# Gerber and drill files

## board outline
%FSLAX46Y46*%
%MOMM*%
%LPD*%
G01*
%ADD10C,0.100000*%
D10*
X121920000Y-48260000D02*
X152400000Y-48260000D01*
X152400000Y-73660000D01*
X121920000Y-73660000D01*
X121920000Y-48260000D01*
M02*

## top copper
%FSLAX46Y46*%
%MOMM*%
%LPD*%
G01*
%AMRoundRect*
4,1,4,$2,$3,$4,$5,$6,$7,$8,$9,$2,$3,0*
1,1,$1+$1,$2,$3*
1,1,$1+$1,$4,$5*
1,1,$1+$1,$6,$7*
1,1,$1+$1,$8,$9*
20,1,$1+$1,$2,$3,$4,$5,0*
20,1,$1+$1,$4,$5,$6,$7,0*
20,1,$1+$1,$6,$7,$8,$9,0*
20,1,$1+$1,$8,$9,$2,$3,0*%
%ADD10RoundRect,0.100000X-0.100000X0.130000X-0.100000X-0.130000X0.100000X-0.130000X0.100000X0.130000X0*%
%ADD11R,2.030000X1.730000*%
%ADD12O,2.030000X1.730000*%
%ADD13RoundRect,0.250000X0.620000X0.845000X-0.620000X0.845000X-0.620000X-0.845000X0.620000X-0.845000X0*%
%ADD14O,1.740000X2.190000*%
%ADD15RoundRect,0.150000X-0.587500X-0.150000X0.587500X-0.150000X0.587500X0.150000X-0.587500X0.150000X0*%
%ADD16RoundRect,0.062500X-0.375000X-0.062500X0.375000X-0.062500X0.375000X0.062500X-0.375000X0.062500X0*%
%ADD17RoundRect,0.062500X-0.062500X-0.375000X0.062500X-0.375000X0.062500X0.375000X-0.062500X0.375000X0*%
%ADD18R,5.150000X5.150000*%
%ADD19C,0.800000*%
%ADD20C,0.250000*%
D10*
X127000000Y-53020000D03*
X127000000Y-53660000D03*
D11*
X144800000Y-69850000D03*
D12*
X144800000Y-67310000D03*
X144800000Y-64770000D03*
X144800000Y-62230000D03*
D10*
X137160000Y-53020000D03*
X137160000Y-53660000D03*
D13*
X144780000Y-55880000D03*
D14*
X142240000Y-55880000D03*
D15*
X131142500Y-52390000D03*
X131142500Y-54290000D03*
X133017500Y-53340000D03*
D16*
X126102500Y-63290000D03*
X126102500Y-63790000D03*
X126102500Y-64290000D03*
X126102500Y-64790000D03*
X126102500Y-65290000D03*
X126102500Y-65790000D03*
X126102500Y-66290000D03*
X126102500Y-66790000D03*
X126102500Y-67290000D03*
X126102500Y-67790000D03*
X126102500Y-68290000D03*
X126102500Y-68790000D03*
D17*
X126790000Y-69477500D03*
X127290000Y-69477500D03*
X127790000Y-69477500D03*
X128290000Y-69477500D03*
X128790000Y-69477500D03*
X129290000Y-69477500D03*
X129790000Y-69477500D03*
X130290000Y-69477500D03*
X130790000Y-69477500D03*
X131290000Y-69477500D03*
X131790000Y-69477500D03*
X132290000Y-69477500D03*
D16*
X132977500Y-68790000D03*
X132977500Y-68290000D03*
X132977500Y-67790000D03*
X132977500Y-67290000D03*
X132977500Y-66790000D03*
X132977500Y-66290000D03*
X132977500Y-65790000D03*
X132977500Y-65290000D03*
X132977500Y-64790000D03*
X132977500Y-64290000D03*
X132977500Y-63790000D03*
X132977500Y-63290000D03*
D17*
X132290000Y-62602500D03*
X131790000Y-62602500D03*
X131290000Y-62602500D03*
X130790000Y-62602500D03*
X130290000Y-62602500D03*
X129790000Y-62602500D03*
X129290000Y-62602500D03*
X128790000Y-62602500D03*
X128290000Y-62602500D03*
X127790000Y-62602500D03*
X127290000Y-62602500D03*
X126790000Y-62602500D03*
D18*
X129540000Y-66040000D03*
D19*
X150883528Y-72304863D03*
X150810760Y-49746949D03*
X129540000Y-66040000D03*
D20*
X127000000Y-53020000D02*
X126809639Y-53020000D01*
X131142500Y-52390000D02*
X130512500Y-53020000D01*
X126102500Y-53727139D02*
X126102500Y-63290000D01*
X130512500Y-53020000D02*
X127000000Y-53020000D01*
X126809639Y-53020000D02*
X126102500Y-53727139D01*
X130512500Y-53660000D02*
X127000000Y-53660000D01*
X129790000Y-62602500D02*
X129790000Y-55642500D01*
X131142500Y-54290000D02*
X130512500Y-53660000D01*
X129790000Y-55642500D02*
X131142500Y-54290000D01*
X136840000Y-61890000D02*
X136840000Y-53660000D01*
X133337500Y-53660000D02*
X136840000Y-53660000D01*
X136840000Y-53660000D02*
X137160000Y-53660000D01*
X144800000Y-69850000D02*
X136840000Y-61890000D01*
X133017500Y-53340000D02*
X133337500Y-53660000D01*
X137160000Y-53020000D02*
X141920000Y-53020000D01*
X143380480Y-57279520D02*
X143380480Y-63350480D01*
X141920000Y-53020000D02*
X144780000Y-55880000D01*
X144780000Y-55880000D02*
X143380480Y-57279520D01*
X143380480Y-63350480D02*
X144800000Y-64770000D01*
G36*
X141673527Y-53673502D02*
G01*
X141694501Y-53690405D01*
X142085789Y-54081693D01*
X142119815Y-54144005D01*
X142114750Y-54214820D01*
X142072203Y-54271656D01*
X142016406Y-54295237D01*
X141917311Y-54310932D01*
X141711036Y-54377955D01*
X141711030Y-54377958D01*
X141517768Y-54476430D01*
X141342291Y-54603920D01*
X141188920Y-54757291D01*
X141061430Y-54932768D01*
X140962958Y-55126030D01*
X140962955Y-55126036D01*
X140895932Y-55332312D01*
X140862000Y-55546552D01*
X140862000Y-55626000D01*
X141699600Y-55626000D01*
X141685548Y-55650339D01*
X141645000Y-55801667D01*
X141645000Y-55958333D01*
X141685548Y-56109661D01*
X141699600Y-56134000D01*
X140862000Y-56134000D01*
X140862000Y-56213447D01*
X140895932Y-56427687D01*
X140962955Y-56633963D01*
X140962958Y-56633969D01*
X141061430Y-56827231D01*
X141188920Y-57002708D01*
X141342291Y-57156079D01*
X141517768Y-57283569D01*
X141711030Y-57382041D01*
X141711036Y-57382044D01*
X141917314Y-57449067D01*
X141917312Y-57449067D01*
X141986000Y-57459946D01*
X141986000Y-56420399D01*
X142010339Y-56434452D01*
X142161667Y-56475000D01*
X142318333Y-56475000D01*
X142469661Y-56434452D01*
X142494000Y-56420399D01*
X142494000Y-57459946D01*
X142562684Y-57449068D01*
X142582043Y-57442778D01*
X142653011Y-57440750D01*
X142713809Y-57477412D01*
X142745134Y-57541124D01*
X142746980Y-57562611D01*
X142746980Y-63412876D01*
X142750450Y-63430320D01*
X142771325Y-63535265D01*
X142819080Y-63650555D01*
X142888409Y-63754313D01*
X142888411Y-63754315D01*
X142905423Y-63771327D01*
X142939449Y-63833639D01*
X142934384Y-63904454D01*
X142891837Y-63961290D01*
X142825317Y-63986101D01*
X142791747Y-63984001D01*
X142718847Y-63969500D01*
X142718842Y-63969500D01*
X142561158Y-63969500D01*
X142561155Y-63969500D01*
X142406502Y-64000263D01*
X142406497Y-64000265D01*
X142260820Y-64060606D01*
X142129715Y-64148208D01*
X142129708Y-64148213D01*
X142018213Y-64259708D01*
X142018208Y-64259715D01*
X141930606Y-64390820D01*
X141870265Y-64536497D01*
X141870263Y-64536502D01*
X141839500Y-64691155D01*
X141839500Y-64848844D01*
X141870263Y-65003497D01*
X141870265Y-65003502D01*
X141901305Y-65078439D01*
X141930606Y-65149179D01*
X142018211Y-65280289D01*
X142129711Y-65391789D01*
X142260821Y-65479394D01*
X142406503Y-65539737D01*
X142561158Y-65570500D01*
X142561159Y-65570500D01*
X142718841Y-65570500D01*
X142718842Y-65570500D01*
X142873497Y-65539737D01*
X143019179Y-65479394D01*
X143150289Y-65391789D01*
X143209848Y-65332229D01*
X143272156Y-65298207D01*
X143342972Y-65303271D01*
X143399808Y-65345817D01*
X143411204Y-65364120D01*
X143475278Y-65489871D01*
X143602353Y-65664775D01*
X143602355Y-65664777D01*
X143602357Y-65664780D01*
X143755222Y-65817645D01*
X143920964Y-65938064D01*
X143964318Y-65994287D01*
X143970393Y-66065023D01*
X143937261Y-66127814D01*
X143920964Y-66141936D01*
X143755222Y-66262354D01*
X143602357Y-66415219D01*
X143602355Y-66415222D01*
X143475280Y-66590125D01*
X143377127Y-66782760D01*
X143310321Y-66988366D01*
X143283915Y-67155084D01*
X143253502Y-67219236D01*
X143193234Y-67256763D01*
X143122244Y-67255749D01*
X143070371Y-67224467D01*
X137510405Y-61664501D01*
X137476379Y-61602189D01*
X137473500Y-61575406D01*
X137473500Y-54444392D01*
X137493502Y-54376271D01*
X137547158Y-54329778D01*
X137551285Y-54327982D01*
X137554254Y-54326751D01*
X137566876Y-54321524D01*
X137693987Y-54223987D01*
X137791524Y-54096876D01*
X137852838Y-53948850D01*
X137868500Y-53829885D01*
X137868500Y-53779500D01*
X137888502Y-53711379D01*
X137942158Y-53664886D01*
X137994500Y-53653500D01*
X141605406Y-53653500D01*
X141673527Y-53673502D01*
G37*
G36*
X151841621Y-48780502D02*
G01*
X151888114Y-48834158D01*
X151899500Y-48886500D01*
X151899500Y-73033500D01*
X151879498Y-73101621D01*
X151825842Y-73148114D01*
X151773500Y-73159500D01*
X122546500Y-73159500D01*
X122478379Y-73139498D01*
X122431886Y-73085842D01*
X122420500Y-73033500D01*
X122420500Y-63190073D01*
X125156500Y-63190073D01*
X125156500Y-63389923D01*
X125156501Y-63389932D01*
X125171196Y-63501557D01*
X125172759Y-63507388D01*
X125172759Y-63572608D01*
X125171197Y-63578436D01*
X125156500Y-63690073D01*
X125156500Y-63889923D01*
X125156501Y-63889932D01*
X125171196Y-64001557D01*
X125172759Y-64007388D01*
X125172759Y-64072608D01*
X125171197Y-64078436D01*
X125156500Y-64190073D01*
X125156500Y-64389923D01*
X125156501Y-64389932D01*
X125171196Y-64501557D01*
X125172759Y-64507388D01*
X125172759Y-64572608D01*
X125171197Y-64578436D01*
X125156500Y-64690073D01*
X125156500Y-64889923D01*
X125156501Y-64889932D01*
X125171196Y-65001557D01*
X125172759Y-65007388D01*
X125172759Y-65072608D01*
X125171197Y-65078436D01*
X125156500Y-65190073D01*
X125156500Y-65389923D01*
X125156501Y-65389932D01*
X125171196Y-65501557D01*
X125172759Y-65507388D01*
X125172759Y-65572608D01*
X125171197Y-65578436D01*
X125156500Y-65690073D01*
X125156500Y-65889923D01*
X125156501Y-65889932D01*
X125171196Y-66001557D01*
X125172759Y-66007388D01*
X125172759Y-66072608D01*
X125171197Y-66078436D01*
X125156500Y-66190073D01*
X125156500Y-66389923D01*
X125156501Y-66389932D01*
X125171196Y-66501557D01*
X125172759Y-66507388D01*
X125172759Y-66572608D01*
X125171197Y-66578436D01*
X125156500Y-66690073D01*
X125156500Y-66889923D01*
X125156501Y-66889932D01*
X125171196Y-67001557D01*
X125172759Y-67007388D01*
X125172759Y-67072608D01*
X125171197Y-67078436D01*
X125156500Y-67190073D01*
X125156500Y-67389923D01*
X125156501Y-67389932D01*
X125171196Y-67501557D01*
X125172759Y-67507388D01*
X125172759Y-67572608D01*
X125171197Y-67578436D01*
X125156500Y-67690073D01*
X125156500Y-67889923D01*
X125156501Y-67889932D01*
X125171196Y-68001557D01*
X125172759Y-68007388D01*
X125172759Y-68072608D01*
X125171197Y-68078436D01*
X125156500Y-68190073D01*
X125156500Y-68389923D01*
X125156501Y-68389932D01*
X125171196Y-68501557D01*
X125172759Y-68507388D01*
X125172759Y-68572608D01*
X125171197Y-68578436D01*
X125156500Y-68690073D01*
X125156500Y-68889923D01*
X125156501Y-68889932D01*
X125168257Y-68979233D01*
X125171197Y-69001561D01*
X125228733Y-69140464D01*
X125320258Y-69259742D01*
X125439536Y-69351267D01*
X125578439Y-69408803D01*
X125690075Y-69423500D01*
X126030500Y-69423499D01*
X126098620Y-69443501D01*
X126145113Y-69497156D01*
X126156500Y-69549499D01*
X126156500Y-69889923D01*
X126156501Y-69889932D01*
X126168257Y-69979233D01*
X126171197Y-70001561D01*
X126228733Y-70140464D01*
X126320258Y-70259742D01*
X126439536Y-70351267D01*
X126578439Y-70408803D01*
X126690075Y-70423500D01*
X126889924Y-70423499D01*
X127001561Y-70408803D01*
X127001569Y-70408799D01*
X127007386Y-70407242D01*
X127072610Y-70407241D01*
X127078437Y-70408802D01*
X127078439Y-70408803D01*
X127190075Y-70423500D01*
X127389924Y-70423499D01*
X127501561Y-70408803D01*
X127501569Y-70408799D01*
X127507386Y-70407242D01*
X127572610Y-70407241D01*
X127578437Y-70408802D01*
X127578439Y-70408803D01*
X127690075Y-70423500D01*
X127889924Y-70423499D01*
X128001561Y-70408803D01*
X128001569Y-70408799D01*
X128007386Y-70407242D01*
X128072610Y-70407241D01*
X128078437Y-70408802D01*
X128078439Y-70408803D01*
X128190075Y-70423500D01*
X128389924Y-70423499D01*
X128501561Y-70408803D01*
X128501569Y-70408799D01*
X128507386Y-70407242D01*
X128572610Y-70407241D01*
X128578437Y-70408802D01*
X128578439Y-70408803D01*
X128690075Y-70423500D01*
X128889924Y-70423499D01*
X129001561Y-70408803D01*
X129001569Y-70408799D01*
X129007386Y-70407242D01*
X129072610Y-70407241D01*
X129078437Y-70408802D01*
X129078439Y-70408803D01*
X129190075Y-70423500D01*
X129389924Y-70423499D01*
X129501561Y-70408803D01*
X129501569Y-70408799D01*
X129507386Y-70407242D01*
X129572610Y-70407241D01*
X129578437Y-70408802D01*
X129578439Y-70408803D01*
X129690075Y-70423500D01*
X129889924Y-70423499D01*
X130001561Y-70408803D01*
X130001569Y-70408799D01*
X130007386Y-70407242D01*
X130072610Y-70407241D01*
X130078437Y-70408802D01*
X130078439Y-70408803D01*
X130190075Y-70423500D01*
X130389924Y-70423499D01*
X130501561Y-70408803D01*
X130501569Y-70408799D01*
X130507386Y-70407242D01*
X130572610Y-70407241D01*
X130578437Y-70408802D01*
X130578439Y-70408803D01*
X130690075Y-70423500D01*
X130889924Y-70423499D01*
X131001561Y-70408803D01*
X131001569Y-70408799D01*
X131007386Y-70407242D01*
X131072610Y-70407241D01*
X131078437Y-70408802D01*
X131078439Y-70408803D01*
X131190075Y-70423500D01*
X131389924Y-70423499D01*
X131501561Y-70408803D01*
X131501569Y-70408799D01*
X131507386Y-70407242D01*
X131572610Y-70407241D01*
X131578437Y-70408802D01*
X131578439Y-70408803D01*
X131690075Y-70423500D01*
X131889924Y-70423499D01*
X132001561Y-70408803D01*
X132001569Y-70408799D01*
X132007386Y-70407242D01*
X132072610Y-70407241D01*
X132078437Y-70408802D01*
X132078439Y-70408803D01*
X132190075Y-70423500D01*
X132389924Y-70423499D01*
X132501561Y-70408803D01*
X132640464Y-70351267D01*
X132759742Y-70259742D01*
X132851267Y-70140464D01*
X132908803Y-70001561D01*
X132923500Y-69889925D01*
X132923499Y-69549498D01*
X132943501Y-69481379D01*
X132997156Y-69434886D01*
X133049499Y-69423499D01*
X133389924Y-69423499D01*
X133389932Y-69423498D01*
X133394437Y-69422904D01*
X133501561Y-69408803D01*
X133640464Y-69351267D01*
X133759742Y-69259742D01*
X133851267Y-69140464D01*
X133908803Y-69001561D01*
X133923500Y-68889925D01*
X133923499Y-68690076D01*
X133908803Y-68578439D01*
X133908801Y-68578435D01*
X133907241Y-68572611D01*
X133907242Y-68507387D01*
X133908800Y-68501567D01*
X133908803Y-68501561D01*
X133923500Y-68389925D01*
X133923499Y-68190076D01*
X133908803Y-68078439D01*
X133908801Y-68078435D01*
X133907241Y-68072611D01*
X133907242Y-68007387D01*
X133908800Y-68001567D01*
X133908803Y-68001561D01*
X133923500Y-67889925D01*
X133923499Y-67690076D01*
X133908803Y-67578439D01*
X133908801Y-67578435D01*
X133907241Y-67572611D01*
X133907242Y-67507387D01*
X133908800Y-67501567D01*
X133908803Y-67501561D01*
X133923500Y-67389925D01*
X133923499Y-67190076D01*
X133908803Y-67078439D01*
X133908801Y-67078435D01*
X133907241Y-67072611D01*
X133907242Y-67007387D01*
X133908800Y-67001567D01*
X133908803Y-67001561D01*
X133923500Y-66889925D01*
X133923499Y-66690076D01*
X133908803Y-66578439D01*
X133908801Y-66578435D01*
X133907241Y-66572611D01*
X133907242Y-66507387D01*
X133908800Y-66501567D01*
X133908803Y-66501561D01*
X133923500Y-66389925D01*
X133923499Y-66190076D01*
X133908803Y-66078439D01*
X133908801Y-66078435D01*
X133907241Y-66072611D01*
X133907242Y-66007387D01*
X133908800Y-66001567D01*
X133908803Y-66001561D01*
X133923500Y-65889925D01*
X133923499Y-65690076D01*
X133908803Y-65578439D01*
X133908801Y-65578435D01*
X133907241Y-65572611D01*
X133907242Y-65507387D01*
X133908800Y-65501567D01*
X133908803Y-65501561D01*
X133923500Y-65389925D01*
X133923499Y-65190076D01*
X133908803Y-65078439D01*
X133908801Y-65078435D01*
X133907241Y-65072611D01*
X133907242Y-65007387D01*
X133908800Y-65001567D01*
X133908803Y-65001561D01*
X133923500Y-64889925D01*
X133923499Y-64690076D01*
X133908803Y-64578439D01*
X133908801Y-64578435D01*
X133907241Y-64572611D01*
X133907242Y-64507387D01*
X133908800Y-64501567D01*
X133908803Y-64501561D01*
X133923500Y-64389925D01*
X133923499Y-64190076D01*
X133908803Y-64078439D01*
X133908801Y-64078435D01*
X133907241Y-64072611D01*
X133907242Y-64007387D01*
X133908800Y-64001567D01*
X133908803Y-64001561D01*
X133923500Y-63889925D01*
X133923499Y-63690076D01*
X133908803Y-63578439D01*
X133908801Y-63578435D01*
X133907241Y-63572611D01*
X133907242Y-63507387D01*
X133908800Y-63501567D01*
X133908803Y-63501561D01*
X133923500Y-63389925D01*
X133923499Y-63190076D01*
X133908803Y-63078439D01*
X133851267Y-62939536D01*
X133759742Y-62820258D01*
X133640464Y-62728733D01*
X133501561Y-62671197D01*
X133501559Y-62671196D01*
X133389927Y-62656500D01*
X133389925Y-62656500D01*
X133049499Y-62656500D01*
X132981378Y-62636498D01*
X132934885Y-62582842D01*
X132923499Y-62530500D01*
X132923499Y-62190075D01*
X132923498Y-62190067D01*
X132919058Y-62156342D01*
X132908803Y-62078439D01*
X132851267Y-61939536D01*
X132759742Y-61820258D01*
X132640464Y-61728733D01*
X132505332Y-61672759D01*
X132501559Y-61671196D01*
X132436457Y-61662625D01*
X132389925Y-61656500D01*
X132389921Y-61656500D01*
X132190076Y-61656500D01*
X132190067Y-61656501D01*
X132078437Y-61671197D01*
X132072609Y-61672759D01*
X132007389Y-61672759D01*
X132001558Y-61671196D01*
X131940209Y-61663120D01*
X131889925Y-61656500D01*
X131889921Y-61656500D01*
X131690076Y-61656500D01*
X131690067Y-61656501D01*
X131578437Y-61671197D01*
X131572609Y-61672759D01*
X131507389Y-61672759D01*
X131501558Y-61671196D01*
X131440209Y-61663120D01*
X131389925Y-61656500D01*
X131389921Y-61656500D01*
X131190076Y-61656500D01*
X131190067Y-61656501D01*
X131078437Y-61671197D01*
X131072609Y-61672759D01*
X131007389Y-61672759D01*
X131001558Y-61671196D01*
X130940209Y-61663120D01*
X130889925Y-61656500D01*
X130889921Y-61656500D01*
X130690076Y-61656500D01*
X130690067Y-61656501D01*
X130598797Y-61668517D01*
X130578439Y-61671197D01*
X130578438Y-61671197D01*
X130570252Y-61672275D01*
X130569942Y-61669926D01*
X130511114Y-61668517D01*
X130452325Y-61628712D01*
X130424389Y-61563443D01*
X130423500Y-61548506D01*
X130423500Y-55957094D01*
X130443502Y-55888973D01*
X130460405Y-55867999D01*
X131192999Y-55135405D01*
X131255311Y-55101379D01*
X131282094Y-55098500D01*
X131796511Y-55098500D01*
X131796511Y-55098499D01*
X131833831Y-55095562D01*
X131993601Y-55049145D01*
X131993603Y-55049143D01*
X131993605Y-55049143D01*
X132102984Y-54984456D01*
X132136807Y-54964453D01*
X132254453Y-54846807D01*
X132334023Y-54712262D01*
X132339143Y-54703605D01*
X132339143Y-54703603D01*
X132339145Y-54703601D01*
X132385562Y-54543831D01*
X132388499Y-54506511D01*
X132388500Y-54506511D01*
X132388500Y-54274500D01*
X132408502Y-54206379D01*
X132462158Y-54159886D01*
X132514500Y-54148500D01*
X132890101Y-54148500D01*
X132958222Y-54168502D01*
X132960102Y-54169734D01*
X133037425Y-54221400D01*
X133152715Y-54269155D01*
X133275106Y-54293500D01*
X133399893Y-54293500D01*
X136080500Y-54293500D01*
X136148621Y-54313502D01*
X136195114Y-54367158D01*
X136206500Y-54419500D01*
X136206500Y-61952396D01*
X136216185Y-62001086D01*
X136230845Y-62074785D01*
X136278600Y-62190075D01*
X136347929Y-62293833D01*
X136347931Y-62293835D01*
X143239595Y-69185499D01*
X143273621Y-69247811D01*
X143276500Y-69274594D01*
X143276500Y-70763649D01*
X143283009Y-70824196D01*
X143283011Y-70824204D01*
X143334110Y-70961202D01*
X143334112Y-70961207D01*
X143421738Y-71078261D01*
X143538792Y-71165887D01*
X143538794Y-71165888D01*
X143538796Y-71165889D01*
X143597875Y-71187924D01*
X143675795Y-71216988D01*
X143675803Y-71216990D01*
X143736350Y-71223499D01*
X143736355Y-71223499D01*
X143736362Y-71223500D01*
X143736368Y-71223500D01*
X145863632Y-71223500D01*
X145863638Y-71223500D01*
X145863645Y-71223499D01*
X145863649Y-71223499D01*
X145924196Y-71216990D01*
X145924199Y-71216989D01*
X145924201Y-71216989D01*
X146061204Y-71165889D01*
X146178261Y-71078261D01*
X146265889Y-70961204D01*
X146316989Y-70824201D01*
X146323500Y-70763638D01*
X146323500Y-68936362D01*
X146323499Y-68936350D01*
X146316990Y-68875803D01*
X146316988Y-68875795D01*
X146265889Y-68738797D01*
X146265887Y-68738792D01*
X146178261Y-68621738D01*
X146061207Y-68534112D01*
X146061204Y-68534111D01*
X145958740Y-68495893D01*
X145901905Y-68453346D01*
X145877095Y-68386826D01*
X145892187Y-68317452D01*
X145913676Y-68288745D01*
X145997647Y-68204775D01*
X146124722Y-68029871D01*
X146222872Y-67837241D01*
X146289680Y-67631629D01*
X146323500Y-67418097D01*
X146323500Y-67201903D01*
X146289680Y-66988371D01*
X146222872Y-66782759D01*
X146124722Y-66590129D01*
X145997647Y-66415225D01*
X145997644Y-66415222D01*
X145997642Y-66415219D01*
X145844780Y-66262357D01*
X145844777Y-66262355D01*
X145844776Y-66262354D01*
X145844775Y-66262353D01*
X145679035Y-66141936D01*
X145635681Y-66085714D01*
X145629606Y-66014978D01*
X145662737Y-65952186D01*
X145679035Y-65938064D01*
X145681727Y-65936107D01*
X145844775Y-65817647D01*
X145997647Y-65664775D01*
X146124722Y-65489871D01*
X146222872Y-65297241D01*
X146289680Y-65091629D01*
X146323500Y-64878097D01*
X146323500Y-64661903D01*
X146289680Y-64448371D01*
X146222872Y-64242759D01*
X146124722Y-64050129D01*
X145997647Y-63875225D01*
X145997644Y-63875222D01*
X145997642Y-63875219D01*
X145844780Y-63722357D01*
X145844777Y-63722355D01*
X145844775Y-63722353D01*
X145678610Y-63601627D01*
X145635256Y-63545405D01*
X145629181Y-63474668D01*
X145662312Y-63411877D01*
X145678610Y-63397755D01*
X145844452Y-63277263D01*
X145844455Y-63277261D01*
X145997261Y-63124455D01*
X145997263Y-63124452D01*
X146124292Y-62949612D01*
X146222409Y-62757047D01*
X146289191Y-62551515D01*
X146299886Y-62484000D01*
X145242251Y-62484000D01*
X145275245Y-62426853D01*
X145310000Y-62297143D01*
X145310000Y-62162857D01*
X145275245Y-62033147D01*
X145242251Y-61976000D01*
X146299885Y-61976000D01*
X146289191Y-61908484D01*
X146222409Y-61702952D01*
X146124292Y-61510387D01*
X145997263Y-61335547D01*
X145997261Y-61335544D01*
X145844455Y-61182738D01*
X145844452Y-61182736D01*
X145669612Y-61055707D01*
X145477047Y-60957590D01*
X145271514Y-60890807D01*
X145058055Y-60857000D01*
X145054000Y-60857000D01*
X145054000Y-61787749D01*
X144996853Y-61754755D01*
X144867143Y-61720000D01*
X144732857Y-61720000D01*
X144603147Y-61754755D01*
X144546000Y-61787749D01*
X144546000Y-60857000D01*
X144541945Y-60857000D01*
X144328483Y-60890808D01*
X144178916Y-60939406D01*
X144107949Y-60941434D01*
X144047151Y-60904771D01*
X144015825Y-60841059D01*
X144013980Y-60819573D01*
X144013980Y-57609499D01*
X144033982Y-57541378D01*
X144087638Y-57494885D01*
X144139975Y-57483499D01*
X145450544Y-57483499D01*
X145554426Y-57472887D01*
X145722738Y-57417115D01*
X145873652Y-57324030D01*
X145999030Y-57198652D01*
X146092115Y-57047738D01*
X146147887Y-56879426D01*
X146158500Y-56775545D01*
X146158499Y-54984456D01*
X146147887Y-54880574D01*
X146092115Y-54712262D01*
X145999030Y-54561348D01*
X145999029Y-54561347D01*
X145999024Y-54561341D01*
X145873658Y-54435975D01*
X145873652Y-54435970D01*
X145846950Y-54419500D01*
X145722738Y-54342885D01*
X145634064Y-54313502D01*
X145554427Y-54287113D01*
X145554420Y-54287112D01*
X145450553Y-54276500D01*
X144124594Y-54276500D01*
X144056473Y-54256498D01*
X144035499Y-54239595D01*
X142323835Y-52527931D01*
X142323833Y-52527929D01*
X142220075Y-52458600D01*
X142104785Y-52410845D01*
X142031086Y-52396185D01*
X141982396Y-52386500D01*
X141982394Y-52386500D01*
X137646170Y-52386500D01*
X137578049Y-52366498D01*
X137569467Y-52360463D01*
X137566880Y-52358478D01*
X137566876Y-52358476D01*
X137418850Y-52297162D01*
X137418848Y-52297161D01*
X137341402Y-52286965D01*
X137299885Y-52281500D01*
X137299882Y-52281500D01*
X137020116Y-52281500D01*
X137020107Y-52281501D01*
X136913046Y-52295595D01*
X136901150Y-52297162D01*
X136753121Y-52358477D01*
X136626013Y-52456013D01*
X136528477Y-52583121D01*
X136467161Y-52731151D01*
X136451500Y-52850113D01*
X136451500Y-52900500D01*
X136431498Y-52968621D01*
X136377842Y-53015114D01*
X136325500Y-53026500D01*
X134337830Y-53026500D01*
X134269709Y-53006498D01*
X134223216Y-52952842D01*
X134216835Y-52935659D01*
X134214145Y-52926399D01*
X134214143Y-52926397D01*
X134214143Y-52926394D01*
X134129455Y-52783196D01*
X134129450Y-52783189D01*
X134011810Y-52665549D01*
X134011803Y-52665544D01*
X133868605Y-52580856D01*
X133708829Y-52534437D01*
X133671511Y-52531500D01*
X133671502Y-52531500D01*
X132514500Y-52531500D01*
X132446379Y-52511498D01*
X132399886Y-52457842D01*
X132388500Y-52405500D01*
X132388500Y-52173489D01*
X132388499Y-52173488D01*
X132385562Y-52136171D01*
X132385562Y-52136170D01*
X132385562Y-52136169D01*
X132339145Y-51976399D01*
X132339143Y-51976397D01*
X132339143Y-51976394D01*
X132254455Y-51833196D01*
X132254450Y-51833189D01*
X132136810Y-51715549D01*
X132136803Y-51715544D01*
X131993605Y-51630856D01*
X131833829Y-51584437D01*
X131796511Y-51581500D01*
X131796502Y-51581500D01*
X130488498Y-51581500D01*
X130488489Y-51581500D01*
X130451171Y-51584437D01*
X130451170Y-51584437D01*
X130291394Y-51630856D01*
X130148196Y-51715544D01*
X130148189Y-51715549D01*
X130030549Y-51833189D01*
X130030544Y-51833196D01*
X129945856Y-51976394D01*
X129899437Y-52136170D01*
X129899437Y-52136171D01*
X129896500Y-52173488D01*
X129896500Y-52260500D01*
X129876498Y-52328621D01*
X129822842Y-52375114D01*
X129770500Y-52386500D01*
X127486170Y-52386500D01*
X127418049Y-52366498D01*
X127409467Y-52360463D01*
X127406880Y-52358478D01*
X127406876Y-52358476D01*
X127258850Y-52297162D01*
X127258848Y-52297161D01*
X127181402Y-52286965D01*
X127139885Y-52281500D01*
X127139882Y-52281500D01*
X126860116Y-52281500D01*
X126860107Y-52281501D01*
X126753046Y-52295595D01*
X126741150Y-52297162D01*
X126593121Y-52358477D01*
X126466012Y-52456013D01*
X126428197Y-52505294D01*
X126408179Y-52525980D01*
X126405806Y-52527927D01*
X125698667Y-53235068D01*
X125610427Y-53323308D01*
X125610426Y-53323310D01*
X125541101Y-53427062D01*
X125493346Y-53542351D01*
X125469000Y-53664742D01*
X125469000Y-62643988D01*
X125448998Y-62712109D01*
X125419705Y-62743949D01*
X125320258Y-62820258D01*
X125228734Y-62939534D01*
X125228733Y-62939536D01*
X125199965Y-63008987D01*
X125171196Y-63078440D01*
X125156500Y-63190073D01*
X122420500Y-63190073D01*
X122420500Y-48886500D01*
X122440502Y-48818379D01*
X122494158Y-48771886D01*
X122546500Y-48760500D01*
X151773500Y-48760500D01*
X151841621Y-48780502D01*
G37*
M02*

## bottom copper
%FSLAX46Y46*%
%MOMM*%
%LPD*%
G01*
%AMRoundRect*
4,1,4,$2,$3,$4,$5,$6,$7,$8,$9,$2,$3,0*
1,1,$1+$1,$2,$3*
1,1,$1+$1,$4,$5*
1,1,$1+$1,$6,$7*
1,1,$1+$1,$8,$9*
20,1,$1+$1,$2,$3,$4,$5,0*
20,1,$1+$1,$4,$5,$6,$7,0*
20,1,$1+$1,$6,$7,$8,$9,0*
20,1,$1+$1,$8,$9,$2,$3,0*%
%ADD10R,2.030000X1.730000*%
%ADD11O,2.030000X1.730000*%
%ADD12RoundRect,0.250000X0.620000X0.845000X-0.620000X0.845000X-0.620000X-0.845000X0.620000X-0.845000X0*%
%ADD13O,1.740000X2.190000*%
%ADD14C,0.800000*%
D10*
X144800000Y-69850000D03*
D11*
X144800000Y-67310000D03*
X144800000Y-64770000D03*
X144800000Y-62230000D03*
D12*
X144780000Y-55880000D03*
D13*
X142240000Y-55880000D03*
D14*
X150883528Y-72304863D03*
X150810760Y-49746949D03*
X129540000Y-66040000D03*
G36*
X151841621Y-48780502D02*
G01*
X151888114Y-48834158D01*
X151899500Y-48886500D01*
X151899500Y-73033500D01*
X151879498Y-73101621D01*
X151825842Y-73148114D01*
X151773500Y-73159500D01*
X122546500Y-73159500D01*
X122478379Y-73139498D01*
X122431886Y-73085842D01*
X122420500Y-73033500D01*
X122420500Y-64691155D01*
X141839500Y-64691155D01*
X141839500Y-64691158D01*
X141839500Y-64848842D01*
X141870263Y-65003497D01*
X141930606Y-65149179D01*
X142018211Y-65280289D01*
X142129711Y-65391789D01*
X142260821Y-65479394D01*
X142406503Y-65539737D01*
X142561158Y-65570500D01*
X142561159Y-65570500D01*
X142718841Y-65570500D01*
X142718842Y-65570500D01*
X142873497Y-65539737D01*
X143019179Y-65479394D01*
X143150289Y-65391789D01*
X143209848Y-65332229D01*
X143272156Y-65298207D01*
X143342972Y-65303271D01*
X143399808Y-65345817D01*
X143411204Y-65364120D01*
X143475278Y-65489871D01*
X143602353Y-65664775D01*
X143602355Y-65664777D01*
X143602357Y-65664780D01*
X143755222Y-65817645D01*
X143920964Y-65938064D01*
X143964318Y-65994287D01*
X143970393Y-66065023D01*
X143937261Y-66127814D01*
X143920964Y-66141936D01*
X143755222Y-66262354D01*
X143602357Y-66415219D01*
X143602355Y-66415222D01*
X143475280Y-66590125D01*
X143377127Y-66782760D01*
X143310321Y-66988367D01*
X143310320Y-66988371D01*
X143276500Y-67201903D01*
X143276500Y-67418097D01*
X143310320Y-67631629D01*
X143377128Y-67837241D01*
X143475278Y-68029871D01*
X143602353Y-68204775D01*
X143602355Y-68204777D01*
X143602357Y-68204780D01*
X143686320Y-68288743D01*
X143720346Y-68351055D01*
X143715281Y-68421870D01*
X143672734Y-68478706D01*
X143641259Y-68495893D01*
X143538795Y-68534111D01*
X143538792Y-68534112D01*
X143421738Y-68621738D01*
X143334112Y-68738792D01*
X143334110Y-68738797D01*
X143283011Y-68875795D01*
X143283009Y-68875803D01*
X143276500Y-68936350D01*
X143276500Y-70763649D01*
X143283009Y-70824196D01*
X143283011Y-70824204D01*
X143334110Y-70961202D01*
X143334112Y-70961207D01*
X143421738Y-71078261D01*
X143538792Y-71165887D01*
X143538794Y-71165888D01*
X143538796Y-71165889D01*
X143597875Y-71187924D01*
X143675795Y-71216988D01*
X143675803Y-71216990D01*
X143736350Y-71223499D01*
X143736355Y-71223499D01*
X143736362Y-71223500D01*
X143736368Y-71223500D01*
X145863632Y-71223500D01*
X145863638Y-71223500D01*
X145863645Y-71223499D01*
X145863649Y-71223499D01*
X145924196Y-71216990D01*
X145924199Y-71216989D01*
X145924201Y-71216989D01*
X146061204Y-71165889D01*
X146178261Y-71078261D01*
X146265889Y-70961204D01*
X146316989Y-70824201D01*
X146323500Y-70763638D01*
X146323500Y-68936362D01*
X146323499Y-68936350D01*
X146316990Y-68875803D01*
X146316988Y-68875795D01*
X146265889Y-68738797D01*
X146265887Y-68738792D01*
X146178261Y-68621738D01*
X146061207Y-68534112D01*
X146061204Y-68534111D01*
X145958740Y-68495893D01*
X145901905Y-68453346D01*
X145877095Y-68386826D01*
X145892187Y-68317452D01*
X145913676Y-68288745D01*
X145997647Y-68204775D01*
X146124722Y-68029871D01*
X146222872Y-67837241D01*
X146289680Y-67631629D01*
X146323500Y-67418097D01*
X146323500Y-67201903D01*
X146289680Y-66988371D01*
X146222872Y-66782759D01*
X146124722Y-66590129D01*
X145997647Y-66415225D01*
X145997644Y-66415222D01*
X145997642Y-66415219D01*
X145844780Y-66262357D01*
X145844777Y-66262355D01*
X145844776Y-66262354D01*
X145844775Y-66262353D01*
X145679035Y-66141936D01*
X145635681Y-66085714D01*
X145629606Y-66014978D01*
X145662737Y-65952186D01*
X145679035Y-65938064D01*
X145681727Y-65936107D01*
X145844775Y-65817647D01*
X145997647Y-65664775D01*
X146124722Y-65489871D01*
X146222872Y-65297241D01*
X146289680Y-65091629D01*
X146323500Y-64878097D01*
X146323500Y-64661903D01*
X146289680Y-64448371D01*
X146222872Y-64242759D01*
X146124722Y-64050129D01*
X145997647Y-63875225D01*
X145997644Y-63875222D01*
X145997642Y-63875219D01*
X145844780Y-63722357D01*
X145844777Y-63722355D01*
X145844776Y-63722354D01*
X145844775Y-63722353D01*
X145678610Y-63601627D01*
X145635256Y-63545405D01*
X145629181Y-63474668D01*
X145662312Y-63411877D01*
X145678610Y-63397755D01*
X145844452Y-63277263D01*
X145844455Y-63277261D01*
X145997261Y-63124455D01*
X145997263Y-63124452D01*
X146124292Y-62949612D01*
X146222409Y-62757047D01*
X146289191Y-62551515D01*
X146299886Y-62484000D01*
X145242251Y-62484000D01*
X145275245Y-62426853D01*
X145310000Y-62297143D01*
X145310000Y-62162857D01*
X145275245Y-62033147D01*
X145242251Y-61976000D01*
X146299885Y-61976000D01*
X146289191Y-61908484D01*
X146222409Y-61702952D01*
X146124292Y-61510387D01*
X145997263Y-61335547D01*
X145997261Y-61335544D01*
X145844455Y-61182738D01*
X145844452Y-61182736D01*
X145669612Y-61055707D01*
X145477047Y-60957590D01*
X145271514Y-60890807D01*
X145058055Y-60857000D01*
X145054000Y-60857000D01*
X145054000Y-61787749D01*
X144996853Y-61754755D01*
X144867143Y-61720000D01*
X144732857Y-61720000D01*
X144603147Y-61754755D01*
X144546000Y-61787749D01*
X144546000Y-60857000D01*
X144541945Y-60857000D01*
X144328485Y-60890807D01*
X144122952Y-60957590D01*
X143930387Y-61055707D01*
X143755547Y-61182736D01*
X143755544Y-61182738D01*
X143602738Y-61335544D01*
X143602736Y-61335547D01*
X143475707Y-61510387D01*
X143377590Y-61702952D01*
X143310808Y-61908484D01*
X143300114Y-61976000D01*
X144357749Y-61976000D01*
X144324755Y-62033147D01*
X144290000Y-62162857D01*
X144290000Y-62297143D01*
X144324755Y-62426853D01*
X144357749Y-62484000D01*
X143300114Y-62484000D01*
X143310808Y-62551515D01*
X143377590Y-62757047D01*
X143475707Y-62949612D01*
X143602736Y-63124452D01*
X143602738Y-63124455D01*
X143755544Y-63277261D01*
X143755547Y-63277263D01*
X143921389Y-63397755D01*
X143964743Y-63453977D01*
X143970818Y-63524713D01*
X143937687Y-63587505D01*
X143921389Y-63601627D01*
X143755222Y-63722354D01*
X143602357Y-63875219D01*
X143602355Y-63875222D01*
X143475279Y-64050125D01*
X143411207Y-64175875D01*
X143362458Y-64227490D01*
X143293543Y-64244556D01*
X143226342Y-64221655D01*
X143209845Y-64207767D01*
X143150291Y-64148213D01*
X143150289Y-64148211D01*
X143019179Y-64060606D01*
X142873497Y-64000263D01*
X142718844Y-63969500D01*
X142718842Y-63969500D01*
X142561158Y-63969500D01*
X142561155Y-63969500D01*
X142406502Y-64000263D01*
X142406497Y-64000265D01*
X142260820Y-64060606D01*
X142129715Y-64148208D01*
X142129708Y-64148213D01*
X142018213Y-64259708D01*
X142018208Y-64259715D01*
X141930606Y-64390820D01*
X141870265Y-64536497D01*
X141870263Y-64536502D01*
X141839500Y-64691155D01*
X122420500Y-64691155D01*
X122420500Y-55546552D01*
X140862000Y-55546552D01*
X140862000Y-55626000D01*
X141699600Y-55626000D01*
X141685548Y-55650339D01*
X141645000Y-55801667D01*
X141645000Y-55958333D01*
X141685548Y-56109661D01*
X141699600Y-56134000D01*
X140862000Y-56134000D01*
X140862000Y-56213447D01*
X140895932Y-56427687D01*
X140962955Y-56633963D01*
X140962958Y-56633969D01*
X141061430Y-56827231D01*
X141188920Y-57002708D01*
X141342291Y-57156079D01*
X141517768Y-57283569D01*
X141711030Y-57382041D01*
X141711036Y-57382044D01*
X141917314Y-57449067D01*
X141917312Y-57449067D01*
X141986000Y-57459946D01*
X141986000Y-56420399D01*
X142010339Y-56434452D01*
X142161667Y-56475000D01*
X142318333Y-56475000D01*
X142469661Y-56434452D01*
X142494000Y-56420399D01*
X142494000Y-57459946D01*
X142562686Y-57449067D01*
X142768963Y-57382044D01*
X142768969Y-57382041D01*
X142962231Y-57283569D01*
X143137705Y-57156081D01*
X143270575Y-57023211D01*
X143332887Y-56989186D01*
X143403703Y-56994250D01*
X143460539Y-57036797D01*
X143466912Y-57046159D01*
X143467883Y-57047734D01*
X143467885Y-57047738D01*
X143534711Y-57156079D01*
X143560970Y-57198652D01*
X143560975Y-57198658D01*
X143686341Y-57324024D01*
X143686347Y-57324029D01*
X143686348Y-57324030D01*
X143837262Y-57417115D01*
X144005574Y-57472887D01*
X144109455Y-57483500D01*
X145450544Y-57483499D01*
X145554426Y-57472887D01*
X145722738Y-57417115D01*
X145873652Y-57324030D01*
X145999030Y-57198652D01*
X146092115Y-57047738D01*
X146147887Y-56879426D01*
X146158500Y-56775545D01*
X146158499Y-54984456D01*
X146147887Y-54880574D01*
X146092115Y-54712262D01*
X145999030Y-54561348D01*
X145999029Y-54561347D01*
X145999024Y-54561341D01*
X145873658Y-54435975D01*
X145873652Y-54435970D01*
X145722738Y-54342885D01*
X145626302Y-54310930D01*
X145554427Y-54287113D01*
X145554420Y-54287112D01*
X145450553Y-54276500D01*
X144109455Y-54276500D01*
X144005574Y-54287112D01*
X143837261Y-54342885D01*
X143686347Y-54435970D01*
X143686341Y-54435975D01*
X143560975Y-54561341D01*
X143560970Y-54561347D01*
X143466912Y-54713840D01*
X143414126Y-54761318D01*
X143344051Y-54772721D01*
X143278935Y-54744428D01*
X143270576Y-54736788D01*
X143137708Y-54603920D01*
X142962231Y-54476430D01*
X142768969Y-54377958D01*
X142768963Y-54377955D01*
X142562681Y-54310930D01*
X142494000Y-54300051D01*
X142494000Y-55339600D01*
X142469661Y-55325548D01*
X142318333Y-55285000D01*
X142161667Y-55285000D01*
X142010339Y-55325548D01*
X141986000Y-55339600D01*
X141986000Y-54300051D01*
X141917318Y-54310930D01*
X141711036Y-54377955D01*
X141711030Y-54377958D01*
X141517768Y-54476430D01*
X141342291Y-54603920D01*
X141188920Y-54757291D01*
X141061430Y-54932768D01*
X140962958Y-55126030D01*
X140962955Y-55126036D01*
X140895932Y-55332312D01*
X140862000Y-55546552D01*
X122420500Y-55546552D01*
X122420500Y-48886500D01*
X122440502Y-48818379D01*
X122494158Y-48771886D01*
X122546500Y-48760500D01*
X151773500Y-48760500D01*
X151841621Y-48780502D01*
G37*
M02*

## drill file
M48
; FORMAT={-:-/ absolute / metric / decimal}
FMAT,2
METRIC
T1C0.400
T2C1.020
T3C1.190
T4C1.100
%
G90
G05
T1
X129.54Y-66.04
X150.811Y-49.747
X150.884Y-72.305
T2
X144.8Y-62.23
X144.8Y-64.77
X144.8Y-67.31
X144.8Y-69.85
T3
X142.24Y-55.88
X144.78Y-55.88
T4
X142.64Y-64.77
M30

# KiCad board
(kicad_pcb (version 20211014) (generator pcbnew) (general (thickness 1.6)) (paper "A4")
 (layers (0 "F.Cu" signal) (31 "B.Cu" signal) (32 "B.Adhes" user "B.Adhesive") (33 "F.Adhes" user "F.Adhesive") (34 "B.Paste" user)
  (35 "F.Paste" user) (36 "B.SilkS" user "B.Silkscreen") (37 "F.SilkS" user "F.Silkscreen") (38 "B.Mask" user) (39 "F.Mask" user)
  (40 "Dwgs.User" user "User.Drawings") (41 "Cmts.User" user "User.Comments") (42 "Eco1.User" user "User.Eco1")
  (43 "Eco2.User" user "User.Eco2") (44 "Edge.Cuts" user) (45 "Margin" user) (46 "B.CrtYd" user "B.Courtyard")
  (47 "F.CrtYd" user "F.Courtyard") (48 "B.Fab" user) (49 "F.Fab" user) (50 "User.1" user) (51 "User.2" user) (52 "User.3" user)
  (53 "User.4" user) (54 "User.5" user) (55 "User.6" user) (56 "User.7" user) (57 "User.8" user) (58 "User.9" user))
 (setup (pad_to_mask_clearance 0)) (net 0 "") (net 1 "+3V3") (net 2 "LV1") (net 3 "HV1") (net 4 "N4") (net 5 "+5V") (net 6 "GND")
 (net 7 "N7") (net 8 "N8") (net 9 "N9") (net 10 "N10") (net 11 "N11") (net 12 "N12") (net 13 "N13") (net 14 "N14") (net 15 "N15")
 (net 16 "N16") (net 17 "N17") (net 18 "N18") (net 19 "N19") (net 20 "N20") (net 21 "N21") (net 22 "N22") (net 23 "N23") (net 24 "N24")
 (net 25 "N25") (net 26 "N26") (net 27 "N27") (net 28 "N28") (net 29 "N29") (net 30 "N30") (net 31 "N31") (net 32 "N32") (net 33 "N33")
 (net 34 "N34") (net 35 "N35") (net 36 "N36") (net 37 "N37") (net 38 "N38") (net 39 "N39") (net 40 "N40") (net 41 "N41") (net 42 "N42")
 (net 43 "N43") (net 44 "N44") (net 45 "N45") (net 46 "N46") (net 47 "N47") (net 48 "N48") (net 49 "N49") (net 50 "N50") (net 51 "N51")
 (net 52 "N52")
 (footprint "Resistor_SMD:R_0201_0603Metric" (layer "F.Cu") (at 127 53.34 -90)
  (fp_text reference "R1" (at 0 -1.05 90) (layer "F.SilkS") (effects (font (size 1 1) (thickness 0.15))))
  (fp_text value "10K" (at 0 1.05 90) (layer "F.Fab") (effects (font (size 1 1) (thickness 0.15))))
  (pad "" smd roundrect locked (at 0.345 0 270) (size 0.318 0.36) (layers "F.Paste") (roundrect_rratio 0.25))
  (pad "" smd roundrect locked (at -0.345 0 270) (size 0.318 0.36) (layers "F.Paste") (roundrect_rratio 0.25))
  (pad "1" smd roundrect locked (at -0.32 0 270) (size 0.46 0.4) (layers "F.Cu" "F.Mask") (roundrect_rratio 0.25) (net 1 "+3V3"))
  (pad "2" smd roundrect locked (at 0.32 0 270) (size 0.46 0.4) (layers "F.Cu" "F.Mask") (roundrect_rratio 0.25) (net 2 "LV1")))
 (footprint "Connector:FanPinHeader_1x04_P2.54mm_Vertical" (layer "F.Cu") (at 144.8 69.85 90)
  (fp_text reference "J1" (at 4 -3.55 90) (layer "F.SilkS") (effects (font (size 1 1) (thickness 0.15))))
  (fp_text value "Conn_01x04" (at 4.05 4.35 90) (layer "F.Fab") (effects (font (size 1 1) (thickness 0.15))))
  (pad "" np_thru_hole circle locked (at 5.08 -2.16 180) (size 1.1 1.1) (drill 1.1) (layers *.Cu *.Mask))
  (pad "1" thru_hole rect locked (at 0 0 180) (size 2.03 1.73) (drill 1.02) (layers *.Cu *.Mask) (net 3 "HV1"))
  (pad "2" thru_hole oval locked (at 2.54 0 180) (size 2.03 1.73) (drill 1.02) (layers *.Cu *.Mask) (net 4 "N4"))
  (pad "3" thru_hole oval locked (at 5.08 0 180) (size 2.03 1.73) (drill 1.02) (layers *.Cu *.Mask) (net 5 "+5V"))
  (pad "4" thru_hole oval locked (at 7.62 0 180) (size 2.03 1.73) (drill 1.02) (layers *.Cu *.Mask) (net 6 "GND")))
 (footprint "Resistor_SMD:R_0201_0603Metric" (layer "F.Cu") (at 137.16 53.34 -90)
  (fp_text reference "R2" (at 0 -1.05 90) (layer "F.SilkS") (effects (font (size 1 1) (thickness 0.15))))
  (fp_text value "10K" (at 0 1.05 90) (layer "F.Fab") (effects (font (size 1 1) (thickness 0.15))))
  (pad "" smd roundrect locked (at 0.345 0 270) (size 0.318 0.36) (layers "F.Paste") (roundrect_rratio 0.25))
  (pad "" smd roundrect locked (at -0.345 0 270) (size 0.318 0.36) (layers "F.Paste") (roundrect_rratio 0.25))
  (pad "1" smd roundrect locked (at -0.32 0 270) (size 0.46 0.4) (layers "F.Cu" "F.Mask") (roundrect_rratio 0.25) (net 5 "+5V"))
  (pad "2" smd roundrect locked (at 0.32 0 270) (size 0.46 0.4) (layers "F.Cu" "F.Mask") (roundrect_rratio 0.25) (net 3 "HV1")))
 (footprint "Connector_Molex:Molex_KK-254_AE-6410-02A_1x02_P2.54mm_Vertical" (layer "F.Cu") (at 144.78 55.88 180)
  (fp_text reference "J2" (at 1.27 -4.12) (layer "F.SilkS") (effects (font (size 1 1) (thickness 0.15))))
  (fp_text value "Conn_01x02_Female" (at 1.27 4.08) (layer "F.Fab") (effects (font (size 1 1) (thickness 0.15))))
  (pad "1" thru_hole roundrect locked (at 0 0 180) (size 1.74 2.19) (drill 1.19) (layers *.Cu *.Mask) (roundrect_rratio 0.143678)
   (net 5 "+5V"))
  (pad "2" thru_hole oval locked (at 2.54 0 180) (size 1.74 2.19) (drill 1.19) (layers *.Cu *.Mask) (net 6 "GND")))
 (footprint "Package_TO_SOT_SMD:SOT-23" (layer "F.Cu") (at 132.08 53.34)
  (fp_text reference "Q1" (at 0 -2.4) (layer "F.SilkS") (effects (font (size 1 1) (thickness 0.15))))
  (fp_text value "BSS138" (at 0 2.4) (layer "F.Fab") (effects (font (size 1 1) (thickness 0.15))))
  (pad "1" smd roundrect locked (at -0.9375 -0.95) (size 1.475 0.6) (layers "F.Cu" "F.Paste" "F.Mask") (roundrect_rratio 0.25)
   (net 1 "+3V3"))
  (pad "2" smd roundrect locked (at -0.9375 0.95) (size 1.475 0.6) (layers "F.Cu" "F.Paste" "F.Mask") (roundrect_rratio 0.25) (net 2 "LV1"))
  (pad "3" smd roundrect locked (at 0.9375 0) (size 1.475 0.6) (layers "F.Cu" "F.Paste" "F.Mask") (roundrect_rratio 0.25) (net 3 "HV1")))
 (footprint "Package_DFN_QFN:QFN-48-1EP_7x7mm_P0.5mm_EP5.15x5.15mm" (layer "F.Cu") (at 129.54 66.04)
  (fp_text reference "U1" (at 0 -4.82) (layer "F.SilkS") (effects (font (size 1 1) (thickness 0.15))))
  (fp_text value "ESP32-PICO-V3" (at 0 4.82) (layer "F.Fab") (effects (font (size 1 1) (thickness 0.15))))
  (pad "" smd roundrect locked (at -1.935 -0.645) (size 1.04 1.04) (layers "F.Paste") (roundrect_rratio 0.240385))
  (pad "" smd roundrect locked (at 1.935 1.935) (size 1.04 1.04) (layers "F.Paste") (roundrect_rratio 0.240385))
  (pad "" smd roundrect locked (at 0.645 0.645) (size 1.04 1.04) (layers "F.Paste") (roundrect_rratio 0.240385))
  (pad "" smd roundrect locked (at -1.935 1.935) (size 1.04 1.04) (layers "F.Paste") (roundrect_rratio 0.240385))
  (pad "" smd roundrect locked (at 1.935 -0.645) (size 1.04 1.04) (layers "F.Paste") (roundrect_rratio 0.240385))
  (pad "" smd roundrect locked (at -0.645 -1.935) (size 1.04 1.04) (layers "F.Paste") (roundrect_rratio 0.240385))
  (pad "" smd roundrect locked (at -0.645 -0.645) (size 1.04 1.04) (layers "F.Paste") (roundrect_rratio 0.240385))
  (pad "" smd roundrect locked (at 1.935 0.645) (size 1.04 1.04) (layers "F.Paste") (roundrect_rratio 0.240385))
  (pad "" smd roundrect locked (at -1.935 0.645) (size 1.04 1.04) (layers "F.Paste") (roundrect_rratio 0.240385))
  (pad "" smd roundrect locked (at 0.645 1.935) (size 1.04 1.04) (layers "F.Paste") (roundrect_rratio 0.240385))
  (pad "" smd roundrect locked (at -0.645 0.645) (size 1.04 1.04) (layers "F.Paste") (roundrect_rratio 0.240385))
  (pad "" smd roundrect locked (at 0.645 -0.645) (size 1.04 1.04) (layers "F.Paste") (roundrect_rratio 0.240385))
  (pad "" smd roundrect locked (at 0.645 -1.935) (size 1.04 1.04) (layers "F.Paste") (roundrect_rratio 0.240385))
  (pad "" smd roundrect locked (at 1.935 -1.935) (size 1.04 1.04) (layers "F.Paste") (roundrect_rratio 0.240385))
  (pad "" smd roundrect locked (at -0.645 1.935) (size 1.04 1.04) (layers "F.Paste") (roundrect_rratio 0.240385))
  (pad "" smd roundrect locked (at -1.935 -1.935) (size 1.04 1.04) (layers "F.Paste") (roundrect_rratio 0.240385))
  (pad "1" smd roundrect locked (at -3.4375 -2.75) (size 0.875 0.25) (layers "F.Cu" "F.Paste" "F.Mask") (roundrect_rratio 0.25)
   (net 1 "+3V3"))
  (pad "2" smd roundrect locked (at -3.4375 -2.25) (size 0.875 0.25) (layers "F.Cu" "F.Paste" "F.Mask") (roundrect_rratio 0.25) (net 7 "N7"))
  (pad "3" smd roundrect locked (at -3.4375 -1.75) (size 0.875 0.25) (layers "F.Cu" "F.Paste" "F.Mask") (roundrect_rratio 0.25) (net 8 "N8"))
  (pad "4" smd roundrect locked (at -3.4375 -1.25) (size 0.875 0.25) (layers "F.Cu" "F.Paste" "F.Mask") (roundrect_rratio 0.25) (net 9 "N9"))
  (pad "5" smd roundrect locked (at -3.4375 -0.75) (size 0.875 0.25) (layers "F.Cu" "F.Paste" "F.Mask") (roundrect_rratio 0.25)
   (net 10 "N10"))
  (pad "6" smd roundrect locked (at -3.4375 -0.25) (size 0.875 0.25) (layers "F.Cu" "F.Paste" "F.Mask") (roundrect_rratio 0.25)
   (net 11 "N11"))
  (pad "7" smd roundrect locked (at -3.4375 0.25) (size 0.875 0.25) (layers "F.Cu" "F.Paste" "F.Mask") (roundrect_rratio 0.25)
   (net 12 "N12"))
  (pad "8" smd roundrect locked (at -3.4375 0.75) (size 0.875 0.25) (layers "F.Cu" "F.Paste" "F.Mask") (roundrect_rratio 0.25)
   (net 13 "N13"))
  (pad "9" smd roundrect locked (at -3.4375 1.25) (size 0.875 0.25) (layers "F.Cu" "F.Paste" "F.Mask") (roundrect_rratio 0.25)
   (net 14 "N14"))
  (pad "10" smd roundrect locked (at -3.4375 1.75) (size 0.875 0.25) (layers "F.Cu" "F.Paste" "F.Mask") (roundrect_rratio 0.25)
   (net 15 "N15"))
  (pad "11" smd roundrect locked (at -3.4375 2.25) (size 0.875 0.25) (layers "F.Cu" "F.Paste" "F.Mask") (roundrect_rratio 0.25)
   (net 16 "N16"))
  (pad "12" smd roundrect locked (at -3.4375 2.75) (size 0.875 0.25) (layers "F.Cu" "F.Paste" "F.Mask") (roundrect_rratio 0.25)
   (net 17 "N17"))
  (pad "13" smd roundrect locked (at -2.75 3.4375) (size 0.25 0.875) (layers "F.Cu" "F.Paste" "F.Mask") (roundrect_rratio 0.25)
   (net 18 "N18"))
  (pad "14" smd roundrect locked (at -2.25 3.4375) (size 0.25 0.875) (layers "F.Cu" "F.Paste" "F.Mask") (roundrect_rratio 0.25)
   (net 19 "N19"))
  (pad "15" smd roundrect locked (at -1.75 3.4375) (size 0.25 0.875) (layers "F.Cu" "F.Paste" "F.Mask") (roundrect_rratio 0.25)
   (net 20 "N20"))
  (pad "16" smd roundrect locked (at -1.25 3.4375) (size 0.25 0.875) (layers "F.Cu" "F.Paste" "F.Mask") (roundrect_rratio 0.25)
   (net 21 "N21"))
  (pad "17" smd roundrect locked (at -0.75 3.4375) (size 0.25 0.875) (layers "F.Cu" "F.Paste" "F.Mask") (roundrect_rratio 0.25)
   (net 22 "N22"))
  (pad "18" smd roundrect locked (at -0.25 3.4375) (size 0.25 0.875) (layers "F.Cu" "F.Paste" "F.Mask") (roundrect_rratio 0.25)
   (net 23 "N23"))
  (pad "19" smd roundrect locked (at 0.25 3.4375) (size 0.25 0.875) (layers "F.Cu" "F.Paste" "F.Mask") (roundrect_rratio 0.25)
   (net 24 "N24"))
  (pad "20" smd roundrect locked (at 0.75 3.4375) (size 0.25 0.875) (layers "F.Cu" "F.Paste" "F.Mask") (roundrect_rratio 0.25)
   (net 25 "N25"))
  (pad "21" smd roundrect locked (at 1.25 3.4375) (size 0.25 0.875) (layers "F.Cu" "F.Paste" "F.Mask") (roundrect_rratio 0.25)
   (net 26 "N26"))
  (pad "22" smd roundrect locked (at 1.75 3.4375) (size 0.25 0.875) (layers "F.Cu" "F.Paste" "F.Mask") (roundrect_rratio 0.25)
   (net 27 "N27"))
  (pad "23" smd roundrect locked (at 2.25 3.4375) (size 0.25 0.875) (layers "F.Cu" "F.Paste" "F.Mask") (roundrect_rratio 0.25)
   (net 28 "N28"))
  (pad "24" smd roundrect locked (at 2.75 3.4375) (size 0.25 0.875) (layers "F.Cu" "F.Paste" "F.Mask") (roundrect_rratio 0.25)
   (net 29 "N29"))
  (pad "25" smd roundrect locked (at 3.4375 2.75) (size 0.875 0.25) (layers "F.Cu" "F.Paste" "F.Mask") (roundrect_rratio 0.25)
   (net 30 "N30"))
  (pad "26" smd roundrect locked (at 3.4375 2.25) (size 0.875 0.25) (layers "F.Cu" "F.Paste" "F.Mask") (roundrect_rratio 0.25)
   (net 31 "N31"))
  (pad "27" smd roundrect locked (at 3.4375 1.75) (size 0.875 0.25) (layers "F.Cu" "F.Paste" "F.Mask") (roundrect_rratio 0.25)
   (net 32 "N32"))
  (pad "28" smd roundrect locked (at 3.4375 1.25) (size 0.875 0.25) (layers "F.Cu" "F.Paste" "F.Mask") (roundrect_rratio 0.25)
   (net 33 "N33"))
  (pad "29" smd roundrect locked (at 3.4375 0.75) (size 0.875 0.25) (layers "F.Cu" "F.Paste" "F.Mask") (roundrect_rratio 0.25)
   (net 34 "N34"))
  (pad "30" smd roundrect locked (at 3.4375 0.25) (size 0.875 0.25) (layers "F.Cu" "F.Paste" "F.Mask") (roundrect_rratio 0.25)
   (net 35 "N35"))
  (pad "31" smd roundrect locked (at 3.4375 -0.25) (size 0.875 0.25) (layers "F.Cu" "F.Paste" "F.Mask") (roundrect_rratio 0.25)
   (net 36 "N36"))
  (pad "32" smd roundrect locked (at 3.4375 -0.75) (size 0.875 0.25) (layers "F.Cu" "F.Paste" "F.Mask") (roundrect_rratio 0.25)
   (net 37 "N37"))
  (pad "33" smd roundrect locked (at 3.4375 -1.25) (size 0.875 0.25) (layers "F.Cu" "F.Paste" "F.Mask") (roundrect_rratio 0.25)
   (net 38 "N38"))
  (pad "34" smd roundrect locked (at 3.4375 -1.75) (size 0.875 0.25) (layers "F.Cu" "F.Paste" "F.Mask") (roundrect_rratio 0.25)
   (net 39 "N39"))
  (pad "35" smd roundrect locked (at 3.4375 -2.25) (size 0.875 0.25) (layers "F.Cu" "F.Paste" "F.Mask") (roundrect_rratio 0.25)
   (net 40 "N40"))
  (pad "36" smd roundrect locked (at 3.4375 -2.75) (size 0.875 0.25) (layers "F.Cu" "F.Paste" "F.Mask") (roundrect_rratio 0.25)
   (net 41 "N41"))
  (pad "37" smd roundrect locked (at 2.75 -3.4375) (size 0.25 0.875) (layers "F.Cu" "F.Paste" "F.Mask") (roundrect_rratio 0.25)
   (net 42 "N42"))
  (pad "38" smd roundrect locked (at 2.25 -3.4375) (size 0.25 0.875) (layers "F.Cu" "F.Paste" "F.Mask") (roundrect_rratio 0.25)
   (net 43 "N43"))
  (pad "39" smd roundrect locked (at 1.75 -3.4375) (size 0.25 0.875) (layers "F.Cu" "F.Paste" "F.Mask") (roundrect_rratio 0.25)
   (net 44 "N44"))
  (pad "40" smd roundrect locked (at 1.25 -3.4375) (size 0.25 0.875) (layers "F.Cu" "F.Paste" "F.Mask") (roundrect_rratio 0.25)
   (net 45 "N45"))
  (pad "41" smd roundrect locked (at 0.75 -3.4375) (size 0.25 0.875) (layers "F.Cu" "F.Paste" "F.Mask") (roundrect_rratio 0.25)
   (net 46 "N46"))
  (pad "42" smd roundrect locked (at 0.25 -3.4375) (size 0.25 0.875) (layers "F.Cu" "F.Paste" "F.Mask") (roundrect_rratio 0.25)
   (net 2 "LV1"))
  (pad "43" smd roundrect locked (at -0.25 -3.4375) (size 0.25 0.875) (layers "F.Cu" "F.Paste" "F.Mask") (roundrect_rratio 0.25)
   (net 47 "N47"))
  (pad "44" smd roundrect locked (at -0.75 -3.4375) (size 0.25 0.875) (layers "F.Cu" "F.Paste" "F.Mask") (roundrect_rratio 0.25)
   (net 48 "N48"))
  (pad "45" smd roundrect locked (at -1.25 -3.4375) (size 0.25 0.875) (layers "F.Cu" "F.Paste" "F.Mask") (roundrect_rratio 0.25)
   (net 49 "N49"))
  (pad "46" smd roundrect locked (at -1.75 -3.4375) (size 0.25 0.875) (layers "F.Cu" "F.Paste" "F.Mask") (roundrect_rratio 0.25)
   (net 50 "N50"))
  (pad "47" smd roundrect locked (at -2.25 -3.4375) (size 0.25 0.875) (layers "F.Cu" "F.Paste" "F.Mask") (roundrect_rratio 0.25)
   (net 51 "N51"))
  (pad "48" smd roundrect locked (at -2.75 -3.4375) (size 0.25 0.875) (layers "F.Cu" "F.Paste" "F.Mask") (roundrect_rratio 0.25)
   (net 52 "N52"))
  (pad "49" smd rect locked (at 0 0) (size 5.15 5.15) (layers "F.Cu" "F.Mask") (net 6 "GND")))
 (gr_rect (start 152.4 73.66) (end 121.92 48.26) (layer "Edge.Cuts") (width 0.1) (fill none))
 (segment (start 127 53.02) (end 126.809639 53.02) (width 0.25) (layer "F.Cu") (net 1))
 (segment (start 131.1425 52.39) (end 130.5125 53.02) (width 0.25) (layer "F.Cu") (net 1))
 (segment (start 126.1025 53.727139) (end 126.1025 63.29) (width 0.25) (layer "F.Cu") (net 1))
 (segment (start 130.5125 53.02) (end 127 53.02) (width 0.25) (layer "F.Cu") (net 1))
 (segment (start 126.809639 53.02) (end 126.1025 53.727139) (width 0.25) (layer "F.Cu") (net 1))
 (segment (start 130.5125 53.66) (end 127 53.66) (width 0.25) (layer "F.Cu") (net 2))
 (segment (start 129.79 62.6025) (end 129.79 55.6425) (width 0.25) (layer "F.Cu") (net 2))
 (segment (start 131.1425 54.29) (end 130.5125 53.66) (width 0.25) (layer "F.Cu") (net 2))
 (segment (start 129.79 55.6425) (end 131.1425 54.29) (width 0.25) (layer "F.Cu") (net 2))
 (segment (start 136.84 61.89) (end 136.84 53.66) (width 0.25) (layer "F.Cu") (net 3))
 (segment (start 133.3375 53.66) (end 136.84 53.66) (width 0.25) (layer "F.Cu") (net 3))
 (segment (start 136.84 53.66) (end 137.16 53.66) (width 0.25) (layer "F.Cu") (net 3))
 (segment (start 144.8 69.85) (end 136.84 61.89) (width 0.25) (layer "F.Cu") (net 3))
 (segment (start 133.0175 53.34) (end 133.3375 53.66) (width 0.25) (layer "F.Cu") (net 3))
 (segment (start 137.16 53.02) (end 141.92 53.02) (width 0.25) (layer "F.Cu") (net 5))
 (segment (start 143.38048 57.27952) (end 143.38048 63.35048) (width 0.25) (layer "F.Cu") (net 5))
 (segment (start 141.92 53.02) (end 144.78 55.88) (width 0.25) (layer "F.Cu") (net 5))
 (segment (start 144.78 55.88) (end 143.38048 57.27952) (width 0.25) (layer "F.Cu") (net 5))
 (segment (start 143.38048 63.35048) (end 144.8 64.77) (width 0.25) (layer "F.Cu") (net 5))
 (via (at 150.883528 72.304863) (size 0.8) (drill 0.4) (layers "F.Cu" "B.Cu") (free) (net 6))
 (via (at 150.81076 49.746949) (size 0.8) (drill 0.4) (layers "F.Cu" "B.Cu") (free) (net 6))
 (via (at 129.54 66.04) (size 0.8) (drill 0.4) (layers "F.Cu" "B.Cu") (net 6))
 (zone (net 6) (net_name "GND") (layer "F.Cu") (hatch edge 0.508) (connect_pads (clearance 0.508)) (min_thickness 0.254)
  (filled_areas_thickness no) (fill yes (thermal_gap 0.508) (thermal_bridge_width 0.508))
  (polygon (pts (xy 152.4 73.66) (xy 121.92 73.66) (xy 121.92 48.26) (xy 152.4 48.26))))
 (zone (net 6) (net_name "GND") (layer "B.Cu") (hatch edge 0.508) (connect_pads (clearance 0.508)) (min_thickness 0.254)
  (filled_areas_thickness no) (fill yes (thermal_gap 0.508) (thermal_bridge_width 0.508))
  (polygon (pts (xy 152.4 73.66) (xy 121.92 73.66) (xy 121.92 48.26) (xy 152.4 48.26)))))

